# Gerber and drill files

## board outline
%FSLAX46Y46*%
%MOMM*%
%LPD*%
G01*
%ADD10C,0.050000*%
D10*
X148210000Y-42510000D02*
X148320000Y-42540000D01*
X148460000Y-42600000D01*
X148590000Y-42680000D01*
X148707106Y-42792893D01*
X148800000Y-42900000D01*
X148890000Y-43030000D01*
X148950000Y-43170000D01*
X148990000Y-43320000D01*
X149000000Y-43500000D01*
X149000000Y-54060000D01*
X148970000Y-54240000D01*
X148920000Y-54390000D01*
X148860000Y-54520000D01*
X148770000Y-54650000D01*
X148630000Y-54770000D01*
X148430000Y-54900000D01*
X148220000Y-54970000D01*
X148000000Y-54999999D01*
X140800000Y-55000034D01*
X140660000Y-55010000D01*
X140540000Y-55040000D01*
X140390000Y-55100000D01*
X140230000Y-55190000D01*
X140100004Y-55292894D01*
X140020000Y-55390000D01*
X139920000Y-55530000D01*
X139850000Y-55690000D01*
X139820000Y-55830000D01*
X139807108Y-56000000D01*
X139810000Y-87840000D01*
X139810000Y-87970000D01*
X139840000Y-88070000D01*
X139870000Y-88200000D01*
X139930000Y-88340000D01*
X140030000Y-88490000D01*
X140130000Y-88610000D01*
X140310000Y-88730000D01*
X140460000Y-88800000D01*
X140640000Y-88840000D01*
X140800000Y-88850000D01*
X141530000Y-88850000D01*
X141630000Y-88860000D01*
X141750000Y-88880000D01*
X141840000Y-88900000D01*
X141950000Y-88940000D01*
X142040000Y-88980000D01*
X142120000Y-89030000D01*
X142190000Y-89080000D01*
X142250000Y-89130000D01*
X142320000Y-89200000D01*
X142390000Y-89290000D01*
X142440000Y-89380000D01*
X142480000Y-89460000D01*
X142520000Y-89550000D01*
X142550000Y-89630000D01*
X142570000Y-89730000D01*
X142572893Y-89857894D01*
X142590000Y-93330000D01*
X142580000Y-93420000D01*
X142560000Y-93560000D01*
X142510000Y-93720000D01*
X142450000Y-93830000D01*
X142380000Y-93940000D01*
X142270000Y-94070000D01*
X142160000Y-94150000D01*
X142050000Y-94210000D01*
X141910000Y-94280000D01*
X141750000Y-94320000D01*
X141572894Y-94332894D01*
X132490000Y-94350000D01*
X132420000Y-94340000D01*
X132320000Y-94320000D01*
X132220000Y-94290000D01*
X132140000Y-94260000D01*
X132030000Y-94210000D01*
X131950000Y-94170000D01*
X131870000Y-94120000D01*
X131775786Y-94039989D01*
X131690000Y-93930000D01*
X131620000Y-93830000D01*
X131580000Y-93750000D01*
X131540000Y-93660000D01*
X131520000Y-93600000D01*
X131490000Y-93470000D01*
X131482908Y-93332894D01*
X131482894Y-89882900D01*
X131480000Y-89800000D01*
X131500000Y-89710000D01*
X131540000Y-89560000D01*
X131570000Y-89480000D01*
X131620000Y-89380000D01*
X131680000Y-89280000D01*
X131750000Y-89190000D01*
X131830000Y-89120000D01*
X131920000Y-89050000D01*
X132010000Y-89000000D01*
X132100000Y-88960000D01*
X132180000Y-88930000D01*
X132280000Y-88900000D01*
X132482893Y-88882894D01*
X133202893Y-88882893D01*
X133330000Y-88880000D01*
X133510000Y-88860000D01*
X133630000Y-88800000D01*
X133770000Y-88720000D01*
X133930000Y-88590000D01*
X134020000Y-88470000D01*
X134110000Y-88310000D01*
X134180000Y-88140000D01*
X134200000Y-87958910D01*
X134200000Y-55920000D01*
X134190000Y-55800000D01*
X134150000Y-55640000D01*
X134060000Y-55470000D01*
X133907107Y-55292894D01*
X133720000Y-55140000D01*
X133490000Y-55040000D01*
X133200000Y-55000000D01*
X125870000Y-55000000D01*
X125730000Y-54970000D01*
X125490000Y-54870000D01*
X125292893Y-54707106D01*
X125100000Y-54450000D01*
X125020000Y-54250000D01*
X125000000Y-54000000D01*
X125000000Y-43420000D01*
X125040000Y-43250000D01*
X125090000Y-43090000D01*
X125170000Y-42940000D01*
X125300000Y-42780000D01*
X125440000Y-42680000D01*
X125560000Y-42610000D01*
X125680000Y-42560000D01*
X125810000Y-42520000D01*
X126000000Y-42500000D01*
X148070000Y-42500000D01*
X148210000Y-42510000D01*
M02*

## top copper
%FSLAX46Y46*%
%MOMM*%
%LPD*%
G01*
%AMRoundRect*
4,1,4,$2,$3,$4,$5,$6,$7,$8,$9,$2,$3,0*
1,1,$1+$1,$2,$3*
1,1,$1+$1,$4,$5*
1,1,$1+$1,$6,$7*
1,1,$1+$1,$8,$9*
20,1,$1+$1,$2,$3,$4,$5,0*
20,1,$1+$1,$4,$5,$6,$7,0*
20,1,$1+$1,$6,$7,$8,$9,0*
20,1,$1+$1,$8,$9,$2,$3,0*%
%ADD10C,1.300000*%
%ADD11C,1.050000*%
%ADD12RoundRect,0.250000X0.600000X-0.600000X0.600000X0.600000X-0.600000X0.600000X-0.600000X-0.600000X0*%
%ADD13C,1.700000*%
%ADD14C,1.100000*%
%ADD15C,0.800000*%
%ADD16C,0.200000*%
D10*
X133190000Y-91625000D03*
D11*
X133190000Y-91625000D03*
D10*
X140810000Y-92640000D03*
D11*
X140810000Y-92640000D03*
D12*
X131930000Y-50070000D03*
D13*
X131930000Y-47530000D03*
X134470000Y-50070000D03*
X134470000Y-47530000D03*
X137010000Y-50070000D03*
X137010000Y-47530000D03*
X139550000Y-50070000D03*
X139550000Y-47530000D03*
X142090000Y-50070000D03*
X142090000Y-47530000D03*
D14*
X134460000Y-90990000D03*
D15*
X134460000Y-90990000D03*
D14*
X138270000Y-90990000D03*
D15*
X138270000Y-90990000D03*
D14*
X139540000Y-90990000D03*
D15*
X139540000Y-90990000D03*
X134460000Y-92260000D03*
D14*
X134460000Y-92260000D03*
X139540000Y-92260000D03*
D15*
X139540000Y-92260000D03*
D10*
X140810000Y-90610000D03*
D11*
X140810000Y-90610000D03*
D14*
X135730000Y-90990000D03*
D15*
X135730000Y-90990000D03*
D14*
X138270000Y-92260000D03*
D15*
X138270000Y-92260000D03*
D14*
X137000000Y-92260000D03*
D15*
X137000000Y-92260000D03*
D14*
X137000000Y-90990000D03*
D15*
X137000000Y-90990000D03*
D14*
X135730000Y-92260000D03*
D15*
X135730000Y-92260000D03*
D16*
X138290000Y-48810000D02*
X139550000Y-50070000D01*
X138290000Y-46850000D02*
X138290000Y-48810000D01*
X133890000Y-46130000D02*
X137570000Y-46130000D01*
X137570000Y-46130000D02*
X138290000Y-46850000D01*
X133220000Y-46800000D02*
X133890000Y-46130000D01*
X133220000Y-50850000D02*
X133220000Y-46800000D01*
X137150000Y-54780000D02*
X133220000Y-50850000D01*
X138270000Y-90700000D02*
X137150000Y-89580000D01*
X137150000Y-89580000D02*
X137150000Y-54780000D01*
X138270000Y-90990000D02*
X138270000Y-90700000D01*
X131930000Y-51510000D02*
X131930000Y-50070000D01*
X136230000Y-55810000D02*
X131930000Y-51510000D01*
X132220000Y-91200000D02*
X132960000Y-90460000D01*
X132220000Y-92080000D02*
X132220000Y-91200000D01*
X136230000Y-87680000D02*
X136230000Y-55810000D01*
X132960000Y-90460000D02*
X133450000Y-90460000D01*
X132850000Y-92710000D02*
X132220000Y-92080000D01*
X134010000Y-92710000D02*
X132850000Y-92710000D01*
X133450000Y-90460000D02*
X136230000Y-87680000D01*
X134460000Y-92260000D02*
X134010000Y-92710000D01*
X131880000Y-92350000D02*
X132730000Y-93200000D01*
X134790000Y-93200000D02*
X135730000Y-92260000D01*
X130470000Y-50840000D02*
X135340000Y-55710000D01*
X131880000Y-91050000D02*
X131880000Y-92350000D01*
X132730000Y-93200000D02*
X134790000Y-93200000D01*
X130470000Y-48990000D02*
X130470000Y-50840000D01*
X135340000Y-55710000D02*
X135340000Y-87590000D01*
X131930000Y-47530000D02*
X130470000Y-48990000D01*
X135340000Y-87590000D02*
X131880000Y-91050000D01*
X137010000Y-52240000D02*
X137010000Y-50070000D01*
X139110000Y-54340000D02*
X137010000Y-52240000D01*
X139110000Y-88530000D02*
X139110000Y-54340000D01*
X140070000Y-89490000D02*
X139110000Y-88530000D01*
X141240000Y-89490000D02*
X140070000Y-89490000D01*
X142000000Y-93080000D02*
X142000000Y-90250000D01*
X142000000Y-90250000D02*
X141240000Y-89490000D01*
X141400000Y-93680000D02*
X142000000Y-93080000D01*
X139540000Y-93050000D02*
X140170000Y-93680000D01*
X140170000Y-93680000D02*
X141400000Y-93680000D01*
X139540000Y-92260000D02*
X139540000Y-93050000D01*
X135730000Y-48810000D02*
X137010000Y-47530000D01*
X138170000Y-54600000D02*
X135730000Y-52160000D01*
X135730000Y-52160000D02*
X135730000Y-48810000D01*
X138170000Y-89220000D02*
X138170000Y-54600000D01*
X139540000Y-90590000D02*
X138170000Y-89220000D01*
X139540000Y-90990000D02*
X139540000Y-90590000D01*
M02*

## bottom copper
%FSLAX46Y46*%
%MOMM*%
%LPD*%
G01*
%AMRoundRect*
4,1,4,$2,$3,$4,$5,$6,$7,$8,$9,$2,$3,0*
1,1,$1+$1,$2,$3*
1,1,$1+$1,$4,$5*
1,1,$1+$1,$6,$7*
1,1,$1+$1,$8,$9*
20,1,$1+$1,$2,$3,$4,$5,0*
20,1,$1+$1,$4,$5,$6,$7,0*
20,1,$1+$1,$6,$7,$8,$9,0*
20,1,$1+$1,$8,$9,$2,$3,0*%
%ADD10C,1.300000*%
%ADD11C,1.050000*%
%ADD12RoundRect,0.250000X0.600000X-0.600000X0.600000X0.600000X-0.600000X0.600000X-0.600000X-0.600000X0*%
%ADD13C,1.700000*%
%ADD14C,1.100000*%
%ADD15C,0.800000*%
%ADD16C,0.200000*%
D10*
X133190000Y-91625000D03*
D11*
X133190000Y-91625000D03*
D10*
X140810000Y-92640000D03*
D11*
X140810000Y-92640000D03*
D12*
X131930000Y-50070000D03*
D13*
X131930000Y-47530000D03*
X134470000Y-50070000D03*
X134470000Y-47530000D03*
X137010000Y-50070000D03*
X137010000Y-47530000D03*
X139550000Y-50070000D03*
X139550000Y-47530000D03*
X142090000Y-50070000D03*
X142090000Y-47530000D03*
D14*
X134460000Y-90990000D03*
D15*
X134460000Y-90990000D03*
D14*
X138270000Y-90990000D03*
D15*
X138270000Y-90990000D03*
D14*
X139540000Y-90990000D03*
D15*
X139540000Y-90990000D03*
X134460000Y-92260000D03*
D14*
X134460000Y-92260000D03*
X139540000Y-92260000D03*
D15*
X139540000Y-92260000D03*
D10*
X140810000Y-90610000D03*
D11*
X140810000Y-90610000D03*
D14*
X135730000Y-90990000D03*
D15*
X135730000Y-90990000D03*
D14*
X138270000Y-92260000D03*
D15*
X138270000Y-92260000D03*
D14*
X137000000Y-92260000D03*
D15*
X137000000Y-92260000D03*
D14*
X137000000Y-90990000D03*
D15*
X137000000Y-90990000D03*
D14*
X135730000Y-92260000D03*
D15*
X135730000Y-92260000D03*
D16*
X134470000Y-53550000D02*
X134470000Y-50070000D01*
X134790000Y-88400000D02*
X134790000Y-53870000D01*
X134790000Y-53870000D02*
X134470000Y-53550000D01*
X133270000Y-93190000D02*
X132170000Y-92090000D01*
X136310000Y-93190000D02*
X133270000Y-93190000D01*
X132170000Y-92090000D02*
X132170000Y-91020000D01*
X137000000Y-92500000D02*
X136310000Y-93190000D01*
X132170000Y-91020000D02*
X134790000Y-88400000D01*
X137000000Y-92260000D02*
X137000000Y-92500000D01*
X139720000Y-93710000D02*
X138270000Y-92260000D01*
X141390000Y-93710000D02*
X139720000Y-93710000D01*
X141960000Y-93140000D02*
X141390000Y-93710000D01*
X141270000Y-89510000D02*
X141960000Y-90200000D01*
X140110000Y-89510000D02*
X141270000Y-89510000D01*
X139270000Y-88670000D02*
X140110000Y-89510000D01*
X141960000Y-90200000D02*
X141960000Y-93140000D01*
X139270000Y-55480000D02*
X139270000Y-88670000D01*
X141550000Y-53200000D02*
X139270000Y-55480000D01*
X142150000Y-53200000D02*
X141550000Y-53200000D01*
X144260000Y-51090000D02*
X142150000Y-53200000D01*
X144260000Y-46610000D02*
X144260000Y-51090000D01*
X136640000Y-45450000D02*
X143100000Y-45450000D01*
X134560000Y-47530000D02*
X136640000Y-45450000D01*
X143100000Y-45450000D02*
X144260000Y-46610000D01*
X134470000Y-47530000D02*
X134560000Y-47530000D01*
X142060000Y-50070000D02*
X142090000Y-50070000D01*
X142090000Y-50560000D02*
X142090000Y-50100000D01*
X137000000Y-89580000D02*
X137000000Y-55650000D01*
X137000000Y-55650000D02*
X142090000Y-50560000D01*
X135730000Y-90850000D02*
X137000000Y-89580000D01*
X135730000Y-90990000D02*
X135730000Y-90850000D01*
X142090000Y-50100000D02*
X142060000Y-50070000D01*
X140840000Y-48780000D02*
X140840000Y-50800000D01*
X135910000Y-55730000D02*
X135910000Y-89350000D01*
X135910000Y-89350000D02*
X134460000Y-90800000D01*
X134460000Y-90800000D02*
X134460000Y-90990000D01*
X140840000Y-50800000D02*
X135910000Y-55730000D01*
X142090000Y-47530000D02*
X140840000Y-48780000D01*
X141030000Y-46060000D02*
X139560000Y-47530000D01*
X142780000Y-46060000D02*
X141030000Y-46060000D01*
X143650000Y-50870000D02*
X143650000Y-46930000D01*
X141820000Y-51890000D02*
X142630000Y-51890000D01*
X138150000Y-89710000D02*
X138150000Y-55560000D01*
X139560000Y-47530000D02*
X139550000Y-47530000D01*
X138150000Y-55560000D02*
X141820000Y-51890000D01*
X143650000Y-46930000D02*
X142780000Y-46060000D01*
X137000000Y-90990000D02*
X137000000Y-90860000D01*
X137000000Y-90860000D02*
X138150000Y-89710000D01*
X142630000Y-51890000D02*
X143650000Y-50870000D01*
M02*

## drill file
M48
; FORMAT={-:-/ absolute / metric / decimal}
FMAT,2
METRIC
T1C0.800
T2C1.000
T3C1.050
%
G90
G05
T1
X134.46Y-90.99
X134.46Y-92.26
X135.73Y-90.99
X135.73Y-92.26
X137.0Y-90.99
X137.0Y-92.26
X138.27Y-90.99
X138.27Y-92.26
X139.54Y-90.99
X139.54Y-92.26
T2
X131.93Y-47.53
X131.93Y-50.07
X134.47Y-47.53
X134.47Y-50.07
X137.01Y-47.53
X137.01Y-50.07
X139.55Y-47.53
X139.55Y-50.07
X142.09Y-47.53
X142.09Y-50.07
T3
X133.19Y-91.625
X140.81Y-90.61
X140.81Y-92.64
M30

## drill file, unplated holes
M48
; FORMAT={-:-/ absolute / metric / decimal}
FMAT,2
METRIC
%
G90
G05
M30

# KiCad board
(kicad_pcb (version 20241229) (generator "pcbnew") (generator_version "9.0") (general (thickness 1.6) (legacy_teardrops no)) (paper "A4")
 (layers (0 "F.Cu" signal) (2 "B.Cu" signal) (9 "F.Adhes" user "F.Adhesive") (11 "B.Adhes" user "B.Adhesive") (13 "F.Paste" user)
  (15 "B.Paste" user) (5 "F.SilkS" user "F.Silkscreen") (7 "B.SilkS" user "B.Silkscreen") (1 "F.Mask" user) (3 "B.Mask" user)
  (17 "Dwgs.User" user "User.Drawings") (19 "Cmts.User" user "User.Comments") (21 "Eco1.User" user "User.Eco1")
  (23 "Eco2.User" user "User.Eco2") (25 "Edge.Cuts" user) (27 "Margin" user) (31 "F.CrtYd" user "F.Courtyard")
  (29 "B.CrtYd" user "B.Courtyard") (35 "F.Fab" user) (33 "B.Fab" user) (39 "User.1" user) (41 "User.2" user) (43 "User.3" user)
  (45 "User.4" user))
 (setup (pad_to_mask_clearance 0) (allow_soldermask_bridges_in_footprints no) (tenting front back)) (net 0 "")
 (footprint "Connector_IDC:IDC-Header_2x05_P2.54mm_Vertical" (layer "F.Cu") (at 131.93 50.07 90)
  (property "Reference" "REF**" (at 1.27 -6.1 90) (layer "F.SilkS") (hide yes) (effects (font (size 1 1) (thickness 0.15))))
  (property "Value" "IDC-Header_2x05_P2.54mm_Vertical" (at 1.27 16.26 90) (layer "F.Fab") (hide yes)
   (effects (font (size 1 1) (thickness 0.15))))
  (pad "1" thru_hole roundrect (at 0 0 90) (size 1.7 1.7) (drill 1) (layers "*.Cu" "*.Mask") (remove_unused_layers no)
   (roundrect_rratio 0.147059))
  (pad "2" thru_hole circle (at 2.54 0 90) (size 1.7 1.7) (drill 1) (layers "*.Cu" "*.Mask") (remove_unused_layers no))
  (pad "3" thru_hole circle (at 0 2.54 90) (size 1.7 1.7) (drill 1) (layers "*.Cu" "*.Mask") (remove_unused_layers no))
  (pad "4" thru_hole circle (at 2.54 2.54 90) (size 1.7 1.7) (drill 1) (layers "*.Cu" "*.Mask") (remove_unused_layers no))
  (pad "5" thru_hole circle (at 0 5.08 90) (size 1.7 1.7) (drill 1) (layers "*.Cu" "*.Mask") (remove_unused_layers no))
  (pad "6" thru_hole circle (at 2.54 5.08 90) (size 1.7 1.7) (drill 1) (layers "*.Cu" "*.Mask") (remove_unused_layers no))
  (pad "7" thru_hole circle (at 0 7.62 90) (size 1.7 1.7) (drill 1) (layers "*.Cu" "*.Mask") (remove_unused_layers no))
  (pad "8" thru_hole circle (at 2.54 7.62 90) (size 1.7 1.7) (drill 1) (layers "*.Cu" "*.Mask") (remove_unused_layers no))
  (pad "9" thru_hole circle (at 0 10.16 90) (size 1.7 1.7) (drill 1) (layers "*.Cu" "*.Mask") (remove_unused_layers no))
  (pad "10" thru_hole circle (at 2.54 10.16 90) (size 1.7 1.7) (drill 1) (layers "*.Cu" "*.Mask") (remove_unused_layers no)))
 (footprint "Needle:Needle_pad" (layer "F.Cu") (at 134.46 90.99)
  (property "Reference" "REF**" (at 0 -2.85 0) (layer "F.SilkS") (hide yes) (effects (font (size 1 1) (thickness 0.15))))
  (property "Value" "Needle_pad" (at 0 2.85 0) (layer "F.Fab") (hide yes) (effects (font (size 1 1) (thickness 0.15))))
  (pad "1" connect circle (at 0 0) (size 1.1 1.1) (layers "F.Cu" "F.Mask") (zone_connect 2))
  (pad "1" connect circle (at 0 0) (size 1.1 1.1) (layers "B.Cu" "B.Mask") (zone_connect 2))
  (pad "10" thru_hole circle (at 0 0) (size 0.8 0.8) (drill 0.8) (layers "*.Cu" "*.Mask") (remove_unused_layers no) (zone_connect 2)))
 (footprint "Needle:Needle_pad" (layer "F.Cu") (at 138.27 90.99)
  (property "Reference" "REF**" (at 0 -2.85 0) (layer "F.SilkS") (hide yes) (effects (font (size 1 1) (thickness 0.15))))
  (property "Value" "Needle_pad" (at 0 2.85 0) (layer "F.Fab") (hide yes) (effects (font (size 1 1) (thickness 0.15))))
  (pad "1" connect circle (at 0 0) (size 1.1 1.1) (layers "F.Cu" "F.Mask") (zone_connect 2))
  (pad "1" connect circle (at 0 0) (size 1.1 1.1) (layers "B.Cu" "B.Mask") (zone_connect 2))
  (pad "7" thru_hole circle (at 0 0) (size 0.8 0.8) (drill 0.8) (layers "*.Cu" "*.Mask") (remove_unused_layers no) (zone_connect 2)))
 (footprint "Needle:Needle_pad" (layer "F.Cu") (at 140.81 92.64)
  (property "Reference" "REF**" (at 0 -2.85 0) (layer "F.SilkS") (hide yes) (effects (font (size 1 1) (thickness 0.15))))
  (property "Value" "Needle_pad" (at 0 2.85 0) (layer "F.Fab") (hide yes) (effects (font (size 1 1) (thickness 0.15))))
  (pad "1" connect circle (at 0 0) (size 1.3 1.3) (layers "F.Cu" "F.Mask") (zone_connect 2))
  (pad "1" connect circle (at 0 0) (size 1.3 1.3) (layers "B.Cu" "B.Mask") (zone_connect 2))
  (pad "NC" thru_hole circle (at 0 0) (size 1.05 1.05) (drill 1.05) (layers "*.Cu" "*.Mask") (remove_unused_layers no) (zone_connect 2)))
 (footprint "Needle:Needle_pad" (layer "F.Cu") (at 139.54 90.99)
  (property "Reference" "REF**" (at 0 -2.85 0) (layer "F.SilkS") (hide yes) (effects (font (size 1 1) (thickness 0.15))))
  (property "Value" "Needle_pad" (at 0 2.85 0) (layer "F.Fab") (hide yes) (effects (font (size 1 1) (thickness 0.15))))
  (pad "1" connect circle (at 0 0) (size 1.1 1.1) (layers "F.Cu" "F.Mask") (zone_connect 2))
  (pad "1" connect circle (at 0 0) (size 1.1 1.1) (layers "B.Cu" "B.Mask") (zone_connect 2))
  (pad "6" thru_hole circle (at 0 0) (size 0.8 0.8) (drill 0.8) (layers "*.Cu" "*.Mask") (remove_unused_layers no) (zone_connect 2)))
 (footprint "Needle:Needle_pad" (layer "F.Cu") (at 134.46 92.26)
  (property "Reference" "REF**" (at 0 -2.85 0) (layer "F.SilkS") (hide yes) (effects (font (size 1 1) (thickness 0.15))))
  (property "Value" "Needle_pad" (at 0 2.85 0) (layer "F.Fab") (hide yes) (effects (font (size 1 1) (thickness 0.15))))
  (pad "1" thru_hole circle (at 0 0) (size 0.8 0.8) (drill 0.8) (layers "*.Cu" "*.Mask") (remove_unused_layers no) (zone_connect 2))
  (pad "1" connect circle (at 0 0) (size 1.1 1.1) (layers "F.Cu" "F.Mask") (zone_connect 2))
  (pad "1" connect circle (at 0 0) (size 1.1 1.1) (layers "B.Cu" "B.Mask") (zone_connect 2)))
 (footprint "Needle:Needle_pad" (layer "F.Cu") (at 139.54 92.26)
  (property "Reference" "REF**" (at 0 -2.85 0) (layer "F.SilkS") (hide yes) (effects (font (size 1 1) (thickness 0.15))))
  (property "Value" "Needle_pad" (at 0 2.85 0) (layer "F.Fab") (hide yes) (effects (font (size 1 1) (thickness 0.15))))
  (pad "1" connect circle (at 0 0) (size 1.1 1.1) (layers "F.Cu" "F.Mask") (zone_connect 2))
  (pad "1" connect circle (at 0 0) (size 1.1 1.1) (layers "B.Cu" "B.Mask") (zone_connect 2))
  (pad "5" thru_hole circle (at 0 0) (size 0.8 0.8) (drill 0.8) (layers "*.Cu" "*.Mask") (remove_unused_layers no) (zone_connect 2)))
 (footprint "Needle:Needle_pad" (layer "F.Cu") (at 133.19 91.625)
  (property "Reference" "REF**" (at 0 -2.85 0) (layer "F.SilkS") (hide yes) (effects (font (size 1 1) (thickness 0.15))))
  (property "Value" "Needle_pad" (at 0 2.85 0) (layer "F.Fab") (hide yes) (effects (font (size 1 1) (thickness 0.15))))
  (pad "1" connect circle (at 0 0) (size 1.3 1.3) (layers "F.Cu" "F.Mask") (zone_connect 2))
  (pad "1" connect circle (at 0 0) (size 1.3 1.3) (layers "B.Cu" "B.Mask") (zone_connect 2))
  (pad "NC" thru_hole circle (at 0 0) (size 1.05 1.05) (drill 1.05) (layers "*.Cu" "*.Mask") (remove_unused_layers no) (zone_connect 2)))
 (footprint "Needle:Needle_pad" (layer "F.Cu") (at 140.81 90.61)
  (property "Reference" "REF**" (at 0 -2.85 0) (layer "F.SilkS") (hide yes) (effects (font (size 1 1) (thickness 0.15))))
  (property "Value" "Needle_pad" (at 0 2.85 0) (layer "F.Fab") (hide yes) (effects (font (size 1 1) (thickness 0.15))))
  (pad "1" connect circle (at 0 0) (size 1.3 1.3) (layers "F.Cu" "F.Mask") (zone_connect 2))
  (pad "1" connect circle (at 0 0) (size 1.3 1.3) (layers "B.Cu" "B.Mask") (zone_connect 2))
  (pad "NC" thru_hole circle (at 0 0) (size 1.05 1.05) (drill 1.05) (layers "*.Cu" "*.Mask") (remove_unused_layers no) (zone_connect 2)))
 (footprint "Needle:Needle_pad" (layer "F.Cu") (at 135.73 90.99)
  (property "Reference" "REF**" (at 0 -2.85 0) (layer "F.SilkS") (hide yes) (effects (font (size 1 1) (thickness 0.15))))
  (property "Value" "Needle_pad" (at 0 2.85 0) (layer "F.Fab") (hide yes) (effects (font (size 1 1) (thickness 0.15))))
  (pad "1" connect circle (at 0 0) (size 1.1 1.1) (layers "F.Cu" "F.Mask") (zone_connect 2))
  (pad "1" connect circle (at 0 0) (size 1.1 1.1) (layers "B.Cu" "B.Mask") (zone_connect 2))
  (pad "9" thru_hole circle (at 0 0) (size 0.8 0.8) (drill 0.8) (layers "*.Cu" "*.Mask") (remove_unused_layers no) (zone_connect 2)))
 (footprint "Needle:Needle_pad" (layer "F.Cu") (at 138.27 92.26)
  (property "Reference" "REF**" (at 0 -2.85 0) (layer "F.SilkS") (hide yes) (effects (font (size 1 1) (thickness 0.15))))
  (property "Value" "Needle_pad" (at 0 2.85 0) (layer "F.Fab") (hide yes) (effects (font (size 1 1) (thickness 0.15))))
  (pad "1" connect circle (at 0 0) (size 1.1 1.1) (layers "F.Cu" "F.Mask") (zone_connect 2))
  (pad "1" connect circle (at 0 0) (size 1.1 1.1) (layers "B.Cu" "B.Mask") (zone_connect 2))
  (pad "4" thru_hole circle (at 0 0) (size 0.8 0.8) (drill 0.8) (layers "*.Cu" "*.Mask") (remove_unused_layers no) (zone_connect 2)))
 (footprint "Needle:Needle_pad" (layer "F.Cu") (at 137 92.26)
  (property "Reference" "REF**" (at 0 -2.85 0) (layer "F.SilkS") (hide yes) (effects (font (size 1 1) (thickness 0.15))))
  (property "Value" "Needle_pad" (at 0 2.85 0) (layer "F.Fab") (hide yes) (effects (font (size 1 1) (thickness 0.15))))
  (pad "1" connect circle (at 0 0) (size 1.1 1.1) (layers "F.Cu" "F.Mask") (zone_connect 2))
  (pad "1" connect circle (at 0 0) (size 1.1 1.1) (layers "B.Cu" "B.Mask") (zone_connect 2))
  (pad "3" thru_hole circle (at 0 0) (size 0.8 0.8) (drill 0.8) (layers "*.Cu" "*.Mask") (remove_unused_layers no) (zone_connect 2)))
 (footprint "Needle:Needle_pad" (layer "F.Cu") (at 137 90.99)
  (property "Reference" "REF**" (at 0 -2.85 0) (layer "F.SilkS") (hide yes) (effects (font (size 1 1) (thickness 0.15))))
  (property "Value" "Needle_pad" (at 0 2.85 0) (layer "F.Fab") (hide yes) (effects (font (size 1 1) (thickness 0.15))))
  (pad "1" connect circle (at 0 0) (size 1.1 1.1) (layers "F.Cu" "F.Mask") (zone_connect 2))
  (pad "1" connect circle (at 0 0) (size 1.1 1.1) (layers "B.Cu" "B.Mask") (zone_connect 2))
  (pad "8" thru_hole circle (at 0 0) (size 0.8 0.8) (drill 0.8) (layers "*.Cu" "*.Mask") (remove_unused_layers no) (zone_connect 2)))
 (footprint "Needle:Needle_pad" (layer "B.Cu") (at 135.73 92.26 180)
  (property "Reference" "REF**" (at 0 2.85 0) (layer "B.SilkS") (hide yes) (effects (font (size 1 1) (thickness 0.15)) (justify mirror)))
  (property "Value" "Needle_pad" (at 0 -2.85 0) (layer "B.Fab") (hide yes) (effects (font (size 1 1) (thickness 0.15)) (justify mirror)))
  (pad "1" connect circle (at 0 0 180) (size 1.1 1.1) (layers "F.Cu" "F.Mask") (zone_connect 2))
  (pad "1" connect circle (at 0 0 180) (size 1.1 1.1) (layers "B.Cu" "B.Mask") (zone_connect 2))
  (pad "2" thru_hole circle (at 0 0 180) (size 0.8 0.8) (drill 0.8) (layers "*.Cu" "*.Mask") (remove_unused_layers no) (zone_connect 2)))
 (gr_poly
  (pts (xy 133.202893 88.882893) (xy 132.482893 88.882894) (xy 132.28 88.9) (xy 132.18 88.93) (xy 132.1 88.96) (xy 132.01 89)
   (xy 131.92 89.05) (xy 131.83 89.12) (xy 131.75 89.19) (xy 131.68 89.28) (xy 131.62 89.38) (xy 131.57 89.48) (xy 131.54 89.56)
   (xy 131.5 89.71) (xy 131.48 89.8) (xy 131.482894 89.8829) (xy 131.482908 93.332894) (xy 131.49 93.47) (xy 131.52 93.6) (xy 131.54 93.66)
   (xy 131.58 93.75) (xy 131.62 93.83) (xy 131.69 93.93) (xy 131.775786 94.039989) (xy 131.87 94.12) (xy 131.95 94.17) (xy 132.03 94.21)
   (xy 132.14 94.26) (xy 132.22 94.29) (xy 132.32 94.32) (xy 132.42 94.34) (xy 132.49 94.35) (xy 141.572894 94.332894) (xy 141.75 94.32)
   (xy 141.91 94.28) (xy 142.05 94.21) (xy 142.16 94.15) (xy 142.27 94.07) (xy 142.38 93.94) (xy 142.45 93.83) (xy 142.51 93.72)
   (xy 142.56 93.56) (xy 142.58 93.42) (xy 142.59 93.33) (xy 142.572893 89.857894) (xy 142.57 89.73) (xy 142.55 89.63) (xy 142.52 89.55)
   (xy 142.48 89.46) (xy 142.44 89.38) (xy 142.39 89.29) (xy 142.32 89.2) (xy 142.25 89.13) (xy 142.19 89.08) (xy 142.12 89.03)
   (xy 142.04 88.98) (xy 141.95 88.94) (xy 141.84 88.9) (xy 141.75 88.88) (xy 141.63 88.86) (xy 141.53 88.85) (xy 140.8 88.85)
   (xy 140.64 88.84) (xy 140.46 88.8) (xy 140.31 88.73) (xy 140.13 88.61) (xy 140.03 88.49) (xy 139.93 88.34) (xy 139.87 88.2)
   (xy 139.84 88.07) (xy 139.81 87.97) (xy 139.81 87.84) (xy 139.807108 56) (xy 139.82 55.83) (xy 139.85 55.69) (xy 139.92 55.53)
   (xy 140.02 55.39) (xy 140.100004 55.292894) (xy 140.23 55.19) (xy 140.39 55.1) (xy 140.54 55.04) (xy 140.66 55.01) (xy 140.8 55.000034)
   (xy 148 54.999999) (xy 148.22 54.97) (xy 148.43 54.9) (xy 148.63 54.77) (xy 148.77 54.65) (xy 148.86 54.52) (xy 148.92 54.39)
   (xy 148.97 54.24) (xy 149 54.06) (xy 149 43.5) (xy 148.99 43.32) (xy 148.95 43.17) (xy 148.89 43.03) (xy 148.8 42.9)
   (xy 148.707106 42.792893) (xy 148.59 42.68) (xy 148.46 42.6) (xy 148.32 42.54) (xy 148.21 42.51) (xy 148.07 42.5) (xy 126 42.5)
   (xy 125.81 42.52) (xy 125.68 42.56) (xy 125.56 42.61) (xy 125.44 42.68) (xy 125.3 42.78) (xy 125.17 42.94) (xy 125.09 43.09)
   (xy 125.04 43.25) (xy 125 43.42) (xy 125 54) (xy 125.02 54.25) (xy 125.1 54.45) (xy 125.292893 54.707106) (xy 125.49 54.87)
   (xy 125.73 54.97) (xy 125.87 55) (xy 133.2 55) (xy 133.49 55.04) (xy 133.72 55.14) (xy 133.907107 55.292894) (xy 134.06 55.47)
   (xy 134.15 55.64) (xy 134.19 55.8) (xy 134.2 55.92) (xy 134.2 87.95891) (xy 134.18 88.14) (xy 134.11 88.31) (xy 134.02 88.47)
   (xy 133.93 88.59) (xy 133.77 88.72) (xy 133.63 88.8) (xy 133.51 88.86) (xy 133.33 88.88))
  (stroke (width 0.05) (type solid)) (fill no) (layer "Edge.Cuts"))
 (segment (start 130.47 48.99) (end 130.47 50.84) (width 0.2) (layer "F.Cu") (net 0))
 (segment (start 131.93 47.53) (end 130.47 48.99) (width 0.2) (layer "F.Cu") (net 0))
 (segment (start 138.29 46.85) (end 138.29 48.81) (width 0.2) (layer "F.Cu") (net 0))
 (segment (start 130.47 50.84) (end 135.34 55.71) (width 0.2) (layer "F.Cu") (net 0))
 (segment (start 132.96 90.46) (end 133.45 90.46) (width 0.2) (layer "F.Cu") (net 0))
 (segment (start 138.27 90.7) (end 137.15 89.58) (width 0.2) (layer "F.Cu") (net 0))
 (segment (start 140.07 89.49) (end 139.11 88.53) (width 0.2) (layer "F.Cu") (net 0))
 (segment (start 133.22 50.85) (end 133.22 46.8) (width 0.2) (layer "F.Cu") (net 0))
 (segment (start 141.24 89.49) (end 140.07 89.49) (width 0.2) (layer "F.Cu") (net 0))
 (segment (start 132.22 91.2) (end 132.96 90.46) (width 0.2) (layer "F.Cu") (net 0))
 (segment (start 138.27 90.99) (end 138.27 90.7) (width 0.2) (layer "F.Cu") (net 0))
 (segment (start 141.4 93.68) (end 142 93.08) (width 0.2) (layer "F.Cu") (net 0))
 (segment (start 139.54 90.59) (end 138.17 89.22) (width 0.2) (layer "F.Cu") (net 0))
 (segment (start 137.15 89.58) (end 137.15 54.78) (width 0.2) (layer "F.Cu") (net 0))
 (segment (start 140.17 93.68) (end 141.4 93.68) (width 0.2) (layer "F.Cu") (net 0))
 (segment (start 132.85 92.71) (end 132.22 92.08) (width 0.2) (layer "F.Cu") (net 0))
 (segment (start 139.54 90.99) (end 139.54 90.59) (width 0.2) (layer "F.Cu") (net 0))
 (segment (start 136.23 55.81) (end 131.93 51.51) (width 0.2) (layer "F.Cu") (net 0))
 (segment (start 132.73 93.2) (end 134.79 93.2) (width 0.2) (layer "F.Cu") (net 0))
 (segment (start 136.23 87.68) (end 136.23 55.81) (width 0.2) (layer "F.Cu") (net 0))
 (segment (start 139.54 92.26) (end 139.54 93.05) (width 0.2) (layer "F.Cu") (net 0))
 (segment (start 134.01 92.71) (end 132.85 92.71) (width 0.2) (layer "F.Cu") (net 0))
 (segment (start 131.88 92.35) (end 132.73 93.2) (width 0.2) (layer "F.Cu") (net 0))
 (segment (start 132.22 92.08) (end 132.22 91.2) (width 0.2) (layer "F.Cu") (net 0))
 (segment (start 135.34 55.71) (end 135.34 87.59) (width 0.2) (layer "F.Cu") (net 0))
 (segment (start 135.73 48.81) (end 137.01 47.53) (width 0.2) (layer "F.Cu") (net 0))
 (segment (start 137.01 52.24) (end 137.01 50.07) (width 0.2) (layer "F.Cu") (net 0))
 (segment (start 137.57 46.13) (end 138.29 46.85) (width 0.2) (layer "F.Cu") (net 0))
 (segment (start 142 93.08) (end 142 90.25) (width 0.2) (layer "F.Cu") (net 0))
 (segment (start 138.17 89.22) (end 138.17 54.6) (width 0.2) (layer "F.Cu") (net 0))
 (segment (start 135.73 52.16) (end 135.73 48.81) (width 0.2) (layer "F.Cu") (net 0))
 (segment (start 138.29 48.81) (end 139.55 50.07) (width 0.2) (layer "F.Cu") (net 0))
 (segment (start 135.34 87.59) (end 131.88 91.05) (width 0.2) (layer "F.Cu") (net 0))
 (segment (start 131.93 51.51) (end 131.93 50.07) (width 0.2) (layer "F.Cu") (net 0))
 (segment (start 139.11 88.53) (end 139.11 54.34) (width 0.2) (layer "F.Cu") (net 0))
 (segment (start 134.79 93.2) (end 135.73 92.26) (width 0.2) (layer "F.Cu") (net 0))
 (segment (start 133.45 90.46) (end 136.23 87.68) (width 0.2) (layer "F.Cu") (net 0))
 (segment (start 138.17 54.6) (end 135.73 52.16) (width 0.2) (layer "F.Cu") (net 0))
 (segment (start 133.22 46.8) (end 133.89 46.13) (width 0.2) (layer "F.Cu") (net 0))
 (segment (start 142 90.25) (end 141.24 89.49) (width 0.2) (layer "F.Cu") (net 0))
 (segment (start 137.15 54.78) (end 133.22 50.85) (width 0.2) (layer "F.Cu") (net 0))
 (segment (start 133.89 46.13) (end 137.57 46.13) (width 0.2) (layer "F.Cu") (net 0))
 (segment (start 139.54 93.05) (end 140.17 93.68) (width 0.2) (layer "F.Cu") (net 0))
 (segment (start 139.11 54.34) (end 137.01 52.24) (width 0.2) (layer "F.Cu") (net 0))
 (segment (start 131.88 91.05) (end 131.88 92.35) (width 0.2) (layer "F.Cu") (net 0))
 (segment (start 134.46 92.26) (end 134.01 92.71) (width 0.2) (layer "F.Cu") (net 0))
 (segment (start 141.03 46.06) (end 139.56 47.53) (width 0.2) (layer "B.Cu") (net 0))
 (segment (start 142.78 46.06) (end 141.03 46.06) (width 0.2) (layer "B.Cu") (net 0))
 (segment (start 142.09 50.56) (end 142.09 50.1) (width 0.2) (layer "B.Cu") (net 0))
 (segment (start 136.64 45.45) (end 143.1 45.45) (width 0.2) (layer "B.Cu") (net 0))
 (segment (start 132.17 91.02) (end 134.79 88.4) (width 0.2) (layer "B.Cu") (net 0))
 (segment (start 140.84 50.8) (end 135.91 55.73) (width 0.2) (layer "B.Cu") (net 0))
 (segment (start 141.55 53.2) (end 139.27 55.48) (width 0.2) (layer "B.Cu") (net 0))
 (segment (start 143.65 50.87) (end 143.65 46.93) (width 0.2) (layer "B.Cu") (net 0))
 (segment (start 134.47 47.53) (end 134.56 47.53) (width 0.2) (layer "B.Cu") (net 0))
 (segment (start 141.82 51.89) (end 142.63 51.89) (width 0.2) (layer "B.Cu") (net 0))
 (segment (start 141.27 89.51) (end 141.96 90.2) (width 0.2) (layer "B.Cu") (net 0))
 (segment (start 139.27 55.48) (end 139.27 88.67) (width 0.2) (layer "B.Cu") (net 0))
 (segment (start 134.79 53.87) (end 134.47 53.55) (width 0.2) (layer "B.Cu") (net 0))
 (segment (start 142.09 50.1) (end 142.06 50.07) (width 0.2) (layer "B.Cu") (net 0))
 (segment (start 139.27 88.67) (end 140.11 89.51) (width 0.2) (layer "B.Cu") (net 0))
 (segment (start 142.09 47.53) (end 140.84 48.78) (width 0.2) (layer "B.Cu") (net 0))
 (segment (start 139.72 93.71) (end 138.27 92.26) (width 0.2) (layer "B.Cu") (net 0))
 (segment (start 141.96 93.14) (end 141.39 93.71) (width 0.2) (layer "B.Cu") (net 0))
 (segment (start 141.96 90.2) (end 141.96 93.14) (width 0.2) (layer "B.Cu") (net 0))
 (segment (start 137 89.58) (end 137 55.65) (width 0.2) (layer "B.Cu") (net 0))
 (segment (start 138.15 89.71) (end 138.15 55.56) (width 0.2) (layer "B.Cu") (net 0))
 (segment (start 144.26 51.09) (end 142.15 53.2) (width 0.2) (layer "B.Cu") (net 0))
 (segment (start 141.39 93.71) (end 139.72 93.71) (width 0.2) (layer "B.Cu") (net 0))
 (segment (start 134.79 88.4) (end 134.79 53.87) (width 0.2) (layer "B.Cu") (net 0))
 (segment (start 132.17 92.09) (end 132.17 91.02) (width 0.2) (layer "B.Cu") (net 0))
 (segment (start 139.56 47.53) (end 139.55 47.53) (width 0.2) (layer "B.Cu") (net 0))
 (segment (start 134.46 90.8) (end 134.46 90.99) (width 0.2) (layer "B.Cu") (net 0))
 (segment (start 143.1 45.45) (end 144.26 46.61) (width 0.2) (layer "B.Cu") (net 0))
 (segment (start 138.15 55.56) (end 141.82 51.89) (width 0.2) (layer "B.Cu") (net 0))
 (segment (start 140.84 48.78) (end 140.84 50.8) (width 0.2) (layer "B.Cu") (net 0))
 (segment (start 135.91 89.35) (end 134.46 90.8) (width 0.2) (layer "B.Cu") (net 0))
 (segment (start 143.65 46.93) (end 142.78 46.06) (width 0.2) (layer "B.Cu") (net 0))
 (segment (start 137 90.99) (end 137 90.86) (width 0.2) (layer "B.Cu") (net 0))
 (segment (start 137 90.86) (end 138.15 89.71) (width 0.2) (layer "B.Cu") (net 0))
 (segment (start 144.26 46.61) (end 144.26 51.09) (width 0.2) (layer "B.Cu") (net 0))
 (segment (start 136.31 93.19) (end 133.27 93.19) (width 0.2) (layer "B.Cu") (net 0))
 (segment (start 142.63 51.89) (end 143.65 50.87) (width 0.2) (layer "B.Cu") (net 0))
 (segment (start 142.06 50.07) (end 142.09 50.07) (width 0.2) (layer "B.Cu") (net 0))
 (segment (start 135.73 90.99) (end 135.73 90.85) (width 0.2) (layer "B.Cu") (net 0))
 (segment (start 142.15 53.2) (end 141.55 53.2) (width 0.2) (layer "B.Cu") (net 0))
 (segment (start 134.47 53.55) (end 134.47 50.07) (width 0.2) (layer "B.Cu") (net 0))
 (segment (start 137 55.65) (end 142.09 50.56) (width 0.2) (layer "B.Cu") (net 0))
 (segment (start 140.11 89.51) (end 141.27 89.51) (width 0.2) (layer "B.Cu") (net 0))
 (segment (start 137 92.26) (end 137 92.5) (width 0.2) (layer "B.Cu") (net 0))
 (segment (start 133.27 93.19) (end 132.17 92.09) (width 0.2) (layer "B.Cu") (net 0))
 (segment (start 134.56 47.53) (end 136.64 45.45) (width 0.2) (layer "B.Cu") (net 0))
 (segment (start 135.91 55.73) (end 135.91 89.35) (width 0.2) (layer "B.Cu") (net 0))
 (segment (start 135.73 90.85) (end 137 89.58) (width 0.2) (layer "B.Cu") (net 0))
 (segment (start 137 92.5) (end 136.31 93.19) (width 0.2) (layer "B.Cu") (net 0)))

